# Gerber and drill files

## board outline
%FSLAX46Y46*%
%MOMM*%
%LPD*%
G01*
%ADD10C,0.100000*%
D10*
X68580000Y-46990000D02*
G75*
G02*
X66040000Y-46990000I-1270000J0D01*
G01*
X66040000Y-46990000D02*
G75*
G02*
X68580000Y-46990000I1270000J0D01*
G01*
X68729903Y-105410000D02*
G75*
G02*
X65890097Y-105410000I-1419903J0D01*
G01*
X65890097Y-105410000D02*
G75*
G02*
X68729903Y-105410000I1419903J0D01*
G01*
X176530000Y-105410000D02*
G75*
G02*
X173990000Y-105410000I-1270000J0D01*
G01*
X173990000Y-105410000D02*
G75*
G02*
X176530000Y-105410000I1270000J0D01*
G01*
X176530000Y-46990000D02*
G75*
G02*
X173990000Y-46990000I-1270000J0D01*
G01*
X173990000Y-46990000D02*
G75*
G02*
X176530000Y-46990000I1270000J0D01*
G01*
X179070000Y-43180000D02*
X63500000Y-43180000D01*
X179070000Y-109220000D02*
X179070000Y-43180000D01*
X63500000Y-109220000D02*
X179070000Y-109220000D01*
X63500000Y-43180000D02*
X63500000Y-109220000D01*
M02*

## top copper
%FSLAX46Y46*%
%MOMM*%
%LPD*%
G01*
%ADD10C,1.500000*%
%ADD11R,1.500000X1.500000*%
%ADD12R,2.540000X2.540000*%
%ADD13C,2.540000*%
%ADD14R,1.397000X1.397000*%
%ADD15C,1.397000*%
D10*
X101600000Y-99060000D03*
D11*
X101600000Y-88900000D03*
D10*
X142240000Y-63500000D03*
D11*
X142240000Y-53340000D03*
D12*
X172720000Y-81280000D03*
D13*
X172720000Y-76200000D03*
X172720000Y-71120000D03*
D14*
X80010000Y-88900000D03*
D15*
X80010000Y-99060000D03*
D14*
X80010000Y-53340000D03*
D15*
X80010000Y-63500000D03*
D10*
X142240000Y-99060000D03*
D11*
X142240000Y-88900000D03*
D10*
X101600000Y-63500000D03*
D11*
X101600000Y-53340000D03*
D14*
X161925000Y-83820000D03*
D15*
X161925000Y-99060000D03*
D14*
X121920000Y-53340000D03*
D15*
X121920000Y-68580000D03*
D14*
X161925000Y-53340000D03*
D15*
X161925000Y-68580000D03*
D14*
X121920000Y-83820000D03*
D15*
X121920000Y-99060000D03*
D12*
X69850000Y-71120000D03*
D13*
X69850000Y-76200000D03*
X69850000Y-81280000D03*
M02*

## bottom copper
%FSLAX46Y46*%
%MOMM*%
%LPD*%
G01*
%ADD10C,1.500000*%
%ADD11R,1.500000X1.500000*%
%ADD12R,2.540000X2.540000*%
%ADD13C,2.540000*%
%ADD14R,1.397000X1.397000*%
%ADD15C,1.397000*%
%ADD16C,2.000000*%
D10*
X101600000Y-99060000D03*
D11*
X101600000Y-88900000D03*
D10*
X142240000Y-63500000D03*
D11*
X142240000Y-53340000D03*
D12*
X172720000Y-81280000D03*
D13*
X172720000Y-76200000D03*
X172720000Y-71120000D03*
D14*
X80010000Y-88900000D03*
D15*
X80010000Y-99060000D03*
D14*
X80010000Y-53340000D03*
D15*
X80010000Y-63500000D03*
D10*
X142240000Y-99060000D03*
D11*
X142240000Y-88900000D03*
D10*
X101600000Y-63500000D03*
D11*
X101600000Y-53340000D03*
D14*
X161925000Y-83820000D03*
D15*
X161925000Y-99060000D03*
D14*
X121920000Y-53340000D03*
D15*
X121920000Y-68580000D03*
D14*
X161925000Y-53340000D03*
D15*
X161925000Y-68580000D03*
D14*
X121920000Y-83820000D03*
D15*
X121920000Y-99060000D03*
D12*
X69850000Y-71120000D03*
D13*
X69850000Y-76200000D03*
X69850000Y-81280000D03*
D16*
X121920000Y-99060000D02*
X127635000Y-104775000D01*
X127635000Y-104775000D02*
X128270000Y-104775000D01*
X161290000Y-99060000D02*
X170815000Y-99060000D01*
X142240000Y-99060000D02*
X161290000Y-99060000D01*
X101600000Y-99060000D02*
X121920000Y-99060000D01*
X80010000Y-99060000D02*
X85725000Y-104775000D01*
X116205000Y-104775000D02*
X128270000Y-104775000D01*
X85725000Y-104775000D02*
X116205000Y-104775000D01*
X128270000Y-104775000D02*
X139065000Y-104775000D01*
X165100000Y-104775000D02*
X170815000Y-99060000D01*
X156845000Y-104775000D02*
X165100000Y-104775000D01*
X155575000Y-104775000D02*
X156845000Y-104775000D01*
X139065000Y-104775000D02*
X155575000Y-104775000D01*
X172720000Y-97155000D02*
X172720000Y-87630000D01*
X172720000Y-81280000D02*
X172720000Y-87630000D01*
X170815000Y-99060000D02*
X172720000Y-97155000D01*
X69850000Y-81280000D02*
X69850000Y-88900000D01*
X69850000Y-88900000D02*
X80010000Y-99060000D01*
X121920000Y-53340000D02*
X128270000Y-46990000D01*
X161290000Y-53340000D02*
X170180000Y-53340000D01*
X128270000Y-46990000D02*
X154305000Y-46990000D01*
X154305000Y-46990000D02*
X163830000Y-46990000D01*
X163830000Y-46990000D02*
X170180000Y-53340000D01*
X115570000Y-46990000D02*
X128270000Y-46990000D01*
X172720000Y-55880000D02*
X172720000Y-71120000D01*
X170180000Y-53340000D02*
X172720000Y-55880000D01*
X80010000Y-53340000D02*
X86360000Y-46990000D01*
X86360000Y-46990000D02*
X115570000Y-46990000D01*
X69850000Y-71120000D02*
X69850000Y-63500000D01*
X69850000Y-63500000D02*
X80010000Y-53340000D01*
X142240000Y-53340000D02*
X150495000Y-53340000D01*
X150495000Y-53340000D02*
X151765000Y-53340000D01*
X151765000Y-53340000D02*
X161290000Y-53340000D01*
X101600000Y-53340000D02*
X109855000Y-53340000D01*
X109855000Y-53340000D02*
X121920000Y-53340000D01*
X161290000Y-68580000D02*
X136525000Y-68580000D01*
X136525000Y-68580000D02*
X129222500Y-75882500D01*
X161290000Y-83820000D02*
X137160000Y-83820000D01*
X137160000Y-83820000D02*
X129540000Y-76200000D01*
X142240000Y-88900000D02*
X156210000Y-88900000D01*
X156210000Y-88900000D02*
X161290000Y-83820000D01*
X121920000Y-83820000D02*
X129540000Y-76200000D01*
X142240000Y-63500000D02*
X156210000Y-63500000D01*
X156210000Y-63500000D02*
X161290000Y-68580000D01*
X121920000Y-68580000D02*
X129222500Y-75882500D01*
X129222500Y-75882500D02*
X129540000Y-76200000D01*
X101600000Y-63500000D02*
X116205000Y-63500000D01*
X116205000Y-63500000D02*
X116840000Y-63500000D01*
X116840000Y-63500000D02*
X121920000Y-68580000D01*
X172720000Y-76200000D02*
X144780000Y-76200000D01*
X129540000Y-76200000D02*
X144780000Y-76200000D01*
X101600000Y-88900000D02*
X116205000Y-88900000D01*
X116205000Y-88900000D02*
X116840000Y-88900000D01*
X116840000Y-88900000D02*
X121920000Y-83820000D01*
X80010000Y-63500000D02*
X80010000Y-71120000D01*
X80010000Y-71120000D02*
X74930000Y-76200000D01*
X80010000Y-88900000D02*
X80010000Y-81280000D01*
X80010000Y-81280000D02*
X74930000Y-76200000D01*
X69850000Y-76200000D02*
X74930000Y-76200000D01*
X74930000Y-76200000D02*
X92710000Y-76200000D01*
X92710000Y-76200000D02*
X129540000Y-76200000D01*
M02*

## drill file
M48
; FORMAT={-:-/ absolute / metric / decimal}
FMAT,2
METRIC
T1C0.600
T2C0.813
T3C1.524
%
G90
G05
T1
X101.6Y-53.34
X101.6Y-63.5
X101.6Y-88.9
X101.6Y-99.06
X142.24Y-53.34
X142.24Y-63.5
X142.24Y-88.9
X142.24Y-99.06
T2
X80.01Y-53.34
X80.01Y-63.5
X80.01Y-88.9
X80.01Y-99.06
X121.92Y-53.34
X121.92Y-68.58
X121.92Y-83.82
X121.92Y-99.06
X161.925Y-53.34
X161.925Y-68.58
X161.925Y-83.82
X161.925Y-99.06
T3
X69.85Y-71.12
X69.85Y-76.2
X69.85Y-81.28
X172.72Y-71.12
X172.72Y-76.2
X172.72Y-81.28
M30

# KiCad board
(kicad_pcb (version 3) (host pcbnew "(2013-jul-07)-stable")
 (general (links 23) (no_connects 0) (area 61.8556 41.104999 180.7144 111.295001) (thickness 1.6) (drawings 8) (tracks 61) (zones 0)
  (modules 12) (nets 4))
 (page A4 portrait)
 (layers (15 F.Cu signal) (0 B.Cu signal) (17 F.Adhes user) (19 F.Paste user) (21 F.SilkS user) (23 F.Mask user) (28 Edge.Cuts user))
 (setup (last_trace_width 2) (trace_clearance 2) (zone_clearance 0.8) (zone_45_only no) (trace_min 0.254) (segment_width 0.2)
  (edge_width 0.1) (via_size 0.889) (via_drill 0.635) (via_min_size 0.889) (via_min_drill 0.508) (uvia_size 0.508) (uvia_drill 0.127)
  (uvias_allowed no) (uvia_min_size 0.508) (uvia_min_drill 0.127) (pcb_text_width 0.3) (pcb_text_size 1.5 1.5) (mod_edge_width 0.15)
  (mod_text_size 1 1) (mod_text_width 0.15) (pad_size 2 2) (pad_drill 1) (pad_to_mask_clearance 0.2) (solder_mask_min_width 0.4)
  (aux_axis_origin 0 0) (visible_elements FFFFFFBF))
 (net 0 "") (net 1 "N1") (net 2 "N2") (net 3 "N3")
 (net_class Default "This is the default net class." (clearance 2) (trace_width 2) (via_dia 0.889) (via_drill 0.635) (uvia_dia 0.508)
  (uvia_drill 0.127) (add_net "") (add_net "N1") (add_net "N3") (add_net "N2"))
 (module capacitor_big (layer F.Cu) (at 104.14 93.98 270)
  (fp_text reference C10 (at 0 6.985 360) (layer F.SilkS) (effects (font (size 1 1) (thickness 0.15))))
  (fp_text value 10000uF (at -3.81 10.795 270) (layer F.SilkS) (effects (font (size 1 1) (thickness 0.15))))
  (pad 2 thru_hole circle (at 5.08 2.54 270) (size 1.5 1.5) (drill 0.6) (layers *.Cu *.Mask F.SilkS) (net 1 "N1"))
  (pad 1 thru_hole rect (at -5.08 2.54 270) (size 1.5 1.5) (drill 0.6) (layers *.Cu *.Mask F.SilkS) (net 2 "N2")))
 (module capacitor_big (layer F.Cu) (at 144.78 58.42 270)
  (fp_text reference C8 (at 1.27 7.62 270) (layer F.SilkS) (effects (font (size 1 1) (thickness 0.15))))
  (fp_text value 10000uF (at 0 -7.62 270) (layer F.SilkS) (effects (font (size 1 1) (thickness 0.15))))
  (pad 2 thru_hole circle (at 5.08 2.54 270) (size 1.5 1.5) (drill 0.6) (layers *.Cu *.Mask F.SilkS) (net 2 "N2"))
  (pad 1 thru_hole rect (at -5.08 2.54 270) (size 1.5 1.5) (drill 0.6) (layers *.Cu *.Mask F.SilkS) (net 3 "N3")))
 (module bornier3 (layer F.Cu) (at 172.72 76.2 90)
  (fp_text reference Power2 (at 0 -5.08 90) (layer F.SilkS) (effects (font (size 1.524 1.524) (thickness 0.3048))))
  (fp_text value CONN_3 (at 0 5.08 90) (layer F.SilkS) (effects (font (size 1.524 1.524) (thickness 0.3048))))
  (pad 1 thru_hole rect (at -5.08 0 90) (size 2.54 2.54) (drill 1.524) (layers *.Cu *.Mask F.SilkS) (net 1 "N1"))
  (pad 2 thru_hole circle (at 0 0 90) (size 2.54 2.54) (drill 1.524) (layers *.Cu *.Mask F.SilkS) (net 2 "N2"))
  (pad 3 thru_hole circle (at 5.08 0 90) (size 2.54 2.54) (drill 1.524) (layers *.Cu *.Mask F.SilkS) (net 3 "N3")))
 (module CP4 (layer F.Cu) (at 80.01 93.98 270)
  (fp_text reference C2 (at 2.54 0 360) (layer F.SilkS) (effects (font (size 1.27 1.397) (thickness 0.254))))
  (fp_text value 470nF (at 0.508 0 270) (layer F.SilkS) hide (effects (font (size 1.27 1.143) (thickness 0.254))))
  (pad 1 thru_hole rect (at -5.08 0 270) (size 1.397 1.397) (drill 0.8128) (layers *.Cu *.Mask F.SilkS) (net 2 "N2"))
  (pad 2 thru_hole circle (at 5.08 0 270) (size 1.397 1.397) (drill 0.8128) (layers *.Cu *.Mask F.SilkS) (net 1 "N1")))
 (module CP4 (layer F.Cu) (at 80.01 58.42 270)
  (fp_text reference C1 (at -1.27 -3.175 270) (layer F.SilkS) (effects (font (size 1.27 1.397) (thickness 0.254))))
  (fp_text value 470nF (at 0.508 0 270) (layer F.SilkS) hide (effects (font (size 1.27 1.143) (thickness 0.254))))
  (pad 1 thru_hole rect (at -5.08 0 270) (size 1.397 1.397) (drill 0.8128) (layers *.Cu *.Mask F.SilkS) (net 3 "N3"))
  (pad 2 thru_hole circle (at 5.08 0 270) (size 1.397 1.397) (drill 0.8128) (layers *.Cu *.Mask F.SilkS) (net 2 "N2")))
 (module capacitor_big (layer F.Cu) (at 144.78 93.98 270)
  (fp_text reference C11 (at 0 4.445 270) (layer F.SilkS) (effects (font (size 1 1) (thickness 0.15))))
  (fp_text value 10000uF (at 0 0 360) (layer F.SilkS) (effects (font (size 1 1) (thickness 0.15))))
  (pad 2 thru_hole circle (at 5.08 2.54 270) (size 1.5 1.5) (drill 0.6) (layers *.Cu *.Mask F.SilkS) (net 1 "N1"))
  (pad 1 thru_hole rect (at -5.08 2.54 270) (size 1.5 1.5) (drill 0.6) (layers *.Cu *.Mask F.SilkS) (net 2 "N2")))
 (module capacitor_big (layer F.Cu) (at 104.14 58.42 270)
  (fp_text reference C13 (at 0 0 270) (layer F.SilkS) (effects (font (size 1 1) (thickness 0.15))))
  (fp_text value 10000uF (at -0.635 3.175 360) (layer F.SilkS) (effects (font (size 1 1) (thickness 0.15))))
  (pad 2 thru_hole circle (at 5.08 2.54 270) (size 1.5 1.5) (drill 0.6) (layers *.Cu *.Mask F.SilkS) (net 2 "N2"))
  (pad 1 thru_hole rect (at -5.08 2.54 270) (size 1.5 1.5) (drill 0.6) (layers *.Cu *.Mask F.SilkS) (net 3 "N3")))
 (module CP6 (layer F.Cu) (at 161.925 91.44 270)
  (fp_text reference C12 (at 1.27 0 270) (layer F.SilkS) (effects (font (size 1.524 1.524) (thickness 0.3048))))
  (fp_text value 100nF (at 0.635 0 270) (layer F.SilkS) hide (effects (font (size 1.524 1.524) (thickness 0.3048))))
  (pad 1 thru_hole rect (at -7.62 0 270) (size 1.397 1.397) (drill 0.8128) (layers *.Cu *.Mask F.SilkS) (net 2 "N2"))
  (pad 2 thru_hole circle (at 7.62 0 270) (size 1.397 1.397) (drill 0.8128) (layers *.Cu *.Mask F.SilkS) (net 1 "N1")))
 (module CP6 (layer F.Cu) (at 121.92 60.96 270)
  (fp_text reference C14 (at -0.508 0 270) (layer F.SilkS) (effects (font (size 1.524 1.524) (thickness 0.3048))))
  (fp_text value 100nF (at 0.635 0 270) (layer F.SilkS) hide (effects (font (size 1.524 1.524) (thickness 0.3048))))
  (pad 1 thru_hole rect (at -7.62 0 270) (size 1.397 1.397) (drill 0.8128) (layers *.Cu *.Mask F.SilkS) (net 3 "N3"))
  (pad 2 thru_hole circle (at 7.62 0 270) (size 1.397 1.397) (drill 0.8128) (layers *.Cu *.Mask F.SilkS) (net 2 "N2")))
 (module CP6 (layer F.Cu) (at 161.925 60.96 270)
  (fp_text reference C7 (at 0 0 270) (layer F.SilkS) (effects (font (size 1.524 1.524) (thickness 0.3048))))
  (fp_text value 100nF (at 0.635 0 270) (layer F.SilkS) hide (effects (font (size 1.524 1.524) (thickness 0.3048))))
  (pad 1 thru_hole rect (at -7.62 0 270) (size 1.397 1.397) (drill 0.8128) (layers *.Cu *.Mask F.SilkS) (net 3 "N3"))
  (pad 2 thru_hole circle (at 7.62 0 270) (size 1.397 1.397) (drill 0.8128) (layers *.Cu *.Mask F.SilkS) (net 2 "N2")))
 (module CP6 (layer F.Cu) (at 121.92 91.44 270)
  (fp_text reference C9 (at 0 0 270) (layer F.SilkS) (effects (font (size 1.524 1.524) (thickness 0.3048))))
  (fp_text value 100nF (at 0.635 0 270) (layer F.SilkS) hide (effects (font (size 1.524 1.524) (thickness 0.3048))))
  (pad 1 thru_hole rect (at -7.62 0 270) (size 1.397 1.397) (drill 0.8128) (layers *.Cu *.Mask F.SilkS) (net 2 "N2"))
  (pad 2 thru_hole circle (at 7.62 0 270) (size 1.397 1.397) (drill 0.8128) (layers *.Cu *.Mask F.SilkS) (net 1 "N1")))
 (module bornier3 (layer F.Cu) (at 69.85 76.2 270)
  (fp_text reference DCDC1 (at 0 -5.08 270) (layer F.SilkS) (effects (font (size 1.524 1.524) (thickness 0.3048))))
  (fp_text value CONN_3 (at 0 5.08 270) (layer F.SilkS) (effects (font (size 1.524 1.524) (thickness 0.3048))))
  (pad 1 thru_hole rect (at -5.08 0 270) (size 2.54 2.54) (drill 1.524) (layers *.Cu *.Mask F.SilkS) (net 3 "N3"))
  (pad 2 thru_hole circle (at 0 0 270) (size 2.54 2.54) (drill 1.524) (layers *.Cu *.Mask F.SilkS) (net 2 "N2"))
  (pad 3 thru_hole circle (at 5.08 0 270) (size 2.54 2.54) (drill 1.524) (layers *.Cu *.Mask F.SilkS) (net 1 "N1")))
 (gr_circle (center 67.31 46.99) (end 68.58 46.99) (layer Edge.Cuts) (width 0.1))
 (gr_circle (center 67.31 105.41) (end 68.58 106.045) (layer Edge.Cuts) (width 0.1))
 (gr_circle (center 175.26 105.41) (end 176.53 105.41) (layer Edge.Cuts) (width 0.1))
 (gr_circle (center 175.26 46.99) (end 176.53 46.99) (layer Edge.Cuts) (width 0.1))
 (gr_line (start 179.07 43.18) (end 63.5 43.18) (angle 90) (layer Edge.Cuts) (width 0.1))
 (gr_line (start 179.07 109.22) (end 179.07 43.18) (angle 90) (layer Edge.Cuts) (width 0.1))
 (gr_line (start 63.5 109.22) (end 179.07 109.22) (angle 90) (layer Edge.Cuts) (width 0.1))
 (gr_line (start 63.5 43.18) (end 63.5 109.22) (angle 90) (layer Edge.Cuts) (width 0.1))
 (segment (start 121.92 99.06) (end 127.635 104.775) (width 2) (layer B.Cu) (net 1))
 (segment (start 127.635 104.775) (end 128.27 104.775) (width 2) (layer B.Cu) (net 1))
 (segment (start 161.29 99.06) (end 170.815 99.06) (width 2) (layer B.Cu) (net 1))
 (segment (start 142.24 99.06) (end 161.29 99.06) (width 2) (layer B.Cu) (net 1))
 (segment (start 101.6 99.06) (end 121.92 99.06) (width 2) (layer B.Cu) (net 1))
 (segment (start 80.01 99.06) (end 85.725 104.775) (width 2) (layer B.Cu) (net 1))
 (segment (start 116.205 104.775) (end 128.27 104.775) (width 2) (layer B.Cu) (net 1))
 (segment (start 85.725 104.775) (end 116.205 104.775) (width 2) (layer B.Cu) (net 1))
 (segment (start 128.27 104.775) (end 139.065 104.775) (width 2) (layer B.Cu) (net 1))
 (segment (start 165.1 104.775) (end 170.815 99.06) (width 2) (layer B.Cu) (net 1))
 (segment (start 156.845 104.775) (end 165.1 104.775) (width 2) (layer B.Cu) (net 1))
 (segment (start 155.575 104.775) (end 156.845 104.775) (width 2) (layer B.Cu) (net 1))
 (segment (start 139.065 104.775) (end 155.575 104.775) (width 2) (layer B.Cu) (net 1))
 (segment (start 172.72 97.155) (end 172.72 87.63) (width 2) (layer B.Cu) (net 1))
 (segment (start 172.72 81.28) (end 172.72 87.63) (width 2) (layer B.Cu) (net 1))
 (segment (start 170.815 99.06) (end 172.72 97.155) (width 2) (layer B.Cu) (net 1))
 (segment (start 69.85 81.28) (end 69.85 88.9) (width 2) (layer B.Cu) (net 1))
 (segment (start 69.85 88.9) (end 80.01 99.06) (width 2) (layer B.Cu) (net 1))
 (segment (start 121.92 53.34) (end 128.27 46.99) (width 2) (layer B.Cu) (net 3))
 (segment (start 161.29 53.34) (end 170.18 53.34) (width 2) (layer B.Cu) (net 3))
 (segment (start 128.27 46.99) (end 154.305 46.99) (width 2) (layer B.Cu) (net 3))
 (segment (start 154.305 46.99) (end 163.83 46.99) (width 2) (layer B.Cu) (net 3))
 (segment (start 163.83 46.99) (end 170.18 53.34) (width 2) (layer B.Cu) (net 3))
 (segment (start 115.57 46.99) (end 128.27 46.99) (width 2) (layer B.Cu) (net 3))
 (segment (start 172.72 55.88) (end 172.72 71.12) (width 2) (layer B.Cu) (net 3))
 (segment (start 170.18 53.34) (end 172.72 55.88) (width 2) (layer B.Cu) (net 3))
 (segment (start 80.01 53.34) (end 86.36 46.99) (width 2) (layer B.Cu) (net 3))
 (segment (start 86.36 46.99) (end 115.57 46.99) (width 2) (layer B.Cu) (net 3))
 (segment (start 69.85 71.12) (end 69.85 63.5) (width 2) (layer B.Cu) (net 3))
 (segment (start 69.85 63.5) (end 80.01 53.34) (width 2) (layer B.Cu) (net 3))
 (segment (start 142.24 53.34) (end 150.495 53.34) (width 2) (layer B.Cu) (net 3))
 (segment (start 150.495 53.34) (end 151.765 53.34) (width 2) (layer B.Cu) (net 3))
 (segment (start 151.765 53.34) (end 161.29 53.34) (width 2) (layer B.Cu) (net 3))
 (segment (start 101.6 53.34) (end 109.855 53.34) (width 2) (layer B.Cu) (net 3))
 (segment (start 109.855 53.34) (end 121.92 53.34) (width 2) (layer B.Cu) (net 3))
 (segment (start 161.29 68.58) (end 136.525 68.58) (width 2) (layer B.Cu) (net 2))
 (segment (start 136.525 68.58) (end 129.2225 75.8825) (width 2) (layer B.Cu) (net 2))
 (segment (start 161.29 83.82) (end 137.16 83.82) (width 2) (layer B.Cu) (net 2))
 (segment (start 137.16 83.82) (end 129.54 76.2) (width 2) (layer B.Cu) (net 2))
 (segment (start 142.24 88.9) (end 156.21 88.9) (width 2) (layer B.Cu) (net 2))
 (segment (start 156.21 88.9) (end 161.29 83.82) (width 2) (layer B.Cu) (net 2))
 (segment (start 121.92 83.82) (end 129.54 76.2) (width 2) (layer B.Cu) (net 2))
 (segment (start 142.24 63.5) (end 156.21 63.5) (width 2) (layer B.Cu) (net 2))
 (segment (start 156.21 63.5) (end 161.29 68.58) (width 2) (layer B.Cu) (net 2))
 (segment (start 121.92 68.58) (end 129.2225 75.8825) (width 2) (layer B.Cu) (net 2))
 (segment (start 129.2225 75.8825) (end 129.54 76.2) (width 2) (layer B.Cu) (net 2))
 (segment (start 101.6 63.5) (end 116.205 63.5) (width 2) (layer B.Cu) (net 2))
 (segment (start 116.205 63.5) (end 116.84 63.5) (width 2) (layer B.Cu) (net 2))
 (segment (start 116.84 63.5) (end 121.92 68.58) (width 2) (layer B.Cu) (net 2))
 (segment (start 172.72 76.2) (end 144.78 76.2) (width 2) (layer B.Cu) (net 2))
 (segment (start 129.54 76.2) (end 144.78 76.2) (width 2) (layer B.Cu) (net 2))
 (segment (start 101.6 88.9) (end 116.205 88.9) (width 2) (layer B.Cu) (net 2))
 (segment (start 116.205 88.9) (end 116.84 88.9) (width 2) (layer B.Cu) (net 2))
 (segment (start 116.84 88.9) (end 121.92 83.82) (width 2) (layer B.Cu) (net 2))
 (segment (start 80.01 63.5) (end 80.01 71.12) (width 2) (layer B.Cu) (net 2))
 (segment (start 80.01 71.12) (end 74.93 76.2) (width 2) (layer B.Cu) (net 2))
 (segment (start 80.01 88.9) (end 80.01 81.28) (width 2) (layer B.Cu) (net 2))
 (segment (start 80.01 81.28) (end 74.93 76.2) (width 2) (layer B.Cu) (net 2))
 (segment (start 69.85 76.2) (end 74.93 76.2) (width 2) (layer B.Cu) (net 2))
 (segment (start 74.93 76.2) (end 92.71 76.2) (width 2) (layer B.Cu) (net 2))
 (segment (start 92.71 76.2) (end 129.54 76.2) (width 2) (layer B.Cu) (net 2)))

